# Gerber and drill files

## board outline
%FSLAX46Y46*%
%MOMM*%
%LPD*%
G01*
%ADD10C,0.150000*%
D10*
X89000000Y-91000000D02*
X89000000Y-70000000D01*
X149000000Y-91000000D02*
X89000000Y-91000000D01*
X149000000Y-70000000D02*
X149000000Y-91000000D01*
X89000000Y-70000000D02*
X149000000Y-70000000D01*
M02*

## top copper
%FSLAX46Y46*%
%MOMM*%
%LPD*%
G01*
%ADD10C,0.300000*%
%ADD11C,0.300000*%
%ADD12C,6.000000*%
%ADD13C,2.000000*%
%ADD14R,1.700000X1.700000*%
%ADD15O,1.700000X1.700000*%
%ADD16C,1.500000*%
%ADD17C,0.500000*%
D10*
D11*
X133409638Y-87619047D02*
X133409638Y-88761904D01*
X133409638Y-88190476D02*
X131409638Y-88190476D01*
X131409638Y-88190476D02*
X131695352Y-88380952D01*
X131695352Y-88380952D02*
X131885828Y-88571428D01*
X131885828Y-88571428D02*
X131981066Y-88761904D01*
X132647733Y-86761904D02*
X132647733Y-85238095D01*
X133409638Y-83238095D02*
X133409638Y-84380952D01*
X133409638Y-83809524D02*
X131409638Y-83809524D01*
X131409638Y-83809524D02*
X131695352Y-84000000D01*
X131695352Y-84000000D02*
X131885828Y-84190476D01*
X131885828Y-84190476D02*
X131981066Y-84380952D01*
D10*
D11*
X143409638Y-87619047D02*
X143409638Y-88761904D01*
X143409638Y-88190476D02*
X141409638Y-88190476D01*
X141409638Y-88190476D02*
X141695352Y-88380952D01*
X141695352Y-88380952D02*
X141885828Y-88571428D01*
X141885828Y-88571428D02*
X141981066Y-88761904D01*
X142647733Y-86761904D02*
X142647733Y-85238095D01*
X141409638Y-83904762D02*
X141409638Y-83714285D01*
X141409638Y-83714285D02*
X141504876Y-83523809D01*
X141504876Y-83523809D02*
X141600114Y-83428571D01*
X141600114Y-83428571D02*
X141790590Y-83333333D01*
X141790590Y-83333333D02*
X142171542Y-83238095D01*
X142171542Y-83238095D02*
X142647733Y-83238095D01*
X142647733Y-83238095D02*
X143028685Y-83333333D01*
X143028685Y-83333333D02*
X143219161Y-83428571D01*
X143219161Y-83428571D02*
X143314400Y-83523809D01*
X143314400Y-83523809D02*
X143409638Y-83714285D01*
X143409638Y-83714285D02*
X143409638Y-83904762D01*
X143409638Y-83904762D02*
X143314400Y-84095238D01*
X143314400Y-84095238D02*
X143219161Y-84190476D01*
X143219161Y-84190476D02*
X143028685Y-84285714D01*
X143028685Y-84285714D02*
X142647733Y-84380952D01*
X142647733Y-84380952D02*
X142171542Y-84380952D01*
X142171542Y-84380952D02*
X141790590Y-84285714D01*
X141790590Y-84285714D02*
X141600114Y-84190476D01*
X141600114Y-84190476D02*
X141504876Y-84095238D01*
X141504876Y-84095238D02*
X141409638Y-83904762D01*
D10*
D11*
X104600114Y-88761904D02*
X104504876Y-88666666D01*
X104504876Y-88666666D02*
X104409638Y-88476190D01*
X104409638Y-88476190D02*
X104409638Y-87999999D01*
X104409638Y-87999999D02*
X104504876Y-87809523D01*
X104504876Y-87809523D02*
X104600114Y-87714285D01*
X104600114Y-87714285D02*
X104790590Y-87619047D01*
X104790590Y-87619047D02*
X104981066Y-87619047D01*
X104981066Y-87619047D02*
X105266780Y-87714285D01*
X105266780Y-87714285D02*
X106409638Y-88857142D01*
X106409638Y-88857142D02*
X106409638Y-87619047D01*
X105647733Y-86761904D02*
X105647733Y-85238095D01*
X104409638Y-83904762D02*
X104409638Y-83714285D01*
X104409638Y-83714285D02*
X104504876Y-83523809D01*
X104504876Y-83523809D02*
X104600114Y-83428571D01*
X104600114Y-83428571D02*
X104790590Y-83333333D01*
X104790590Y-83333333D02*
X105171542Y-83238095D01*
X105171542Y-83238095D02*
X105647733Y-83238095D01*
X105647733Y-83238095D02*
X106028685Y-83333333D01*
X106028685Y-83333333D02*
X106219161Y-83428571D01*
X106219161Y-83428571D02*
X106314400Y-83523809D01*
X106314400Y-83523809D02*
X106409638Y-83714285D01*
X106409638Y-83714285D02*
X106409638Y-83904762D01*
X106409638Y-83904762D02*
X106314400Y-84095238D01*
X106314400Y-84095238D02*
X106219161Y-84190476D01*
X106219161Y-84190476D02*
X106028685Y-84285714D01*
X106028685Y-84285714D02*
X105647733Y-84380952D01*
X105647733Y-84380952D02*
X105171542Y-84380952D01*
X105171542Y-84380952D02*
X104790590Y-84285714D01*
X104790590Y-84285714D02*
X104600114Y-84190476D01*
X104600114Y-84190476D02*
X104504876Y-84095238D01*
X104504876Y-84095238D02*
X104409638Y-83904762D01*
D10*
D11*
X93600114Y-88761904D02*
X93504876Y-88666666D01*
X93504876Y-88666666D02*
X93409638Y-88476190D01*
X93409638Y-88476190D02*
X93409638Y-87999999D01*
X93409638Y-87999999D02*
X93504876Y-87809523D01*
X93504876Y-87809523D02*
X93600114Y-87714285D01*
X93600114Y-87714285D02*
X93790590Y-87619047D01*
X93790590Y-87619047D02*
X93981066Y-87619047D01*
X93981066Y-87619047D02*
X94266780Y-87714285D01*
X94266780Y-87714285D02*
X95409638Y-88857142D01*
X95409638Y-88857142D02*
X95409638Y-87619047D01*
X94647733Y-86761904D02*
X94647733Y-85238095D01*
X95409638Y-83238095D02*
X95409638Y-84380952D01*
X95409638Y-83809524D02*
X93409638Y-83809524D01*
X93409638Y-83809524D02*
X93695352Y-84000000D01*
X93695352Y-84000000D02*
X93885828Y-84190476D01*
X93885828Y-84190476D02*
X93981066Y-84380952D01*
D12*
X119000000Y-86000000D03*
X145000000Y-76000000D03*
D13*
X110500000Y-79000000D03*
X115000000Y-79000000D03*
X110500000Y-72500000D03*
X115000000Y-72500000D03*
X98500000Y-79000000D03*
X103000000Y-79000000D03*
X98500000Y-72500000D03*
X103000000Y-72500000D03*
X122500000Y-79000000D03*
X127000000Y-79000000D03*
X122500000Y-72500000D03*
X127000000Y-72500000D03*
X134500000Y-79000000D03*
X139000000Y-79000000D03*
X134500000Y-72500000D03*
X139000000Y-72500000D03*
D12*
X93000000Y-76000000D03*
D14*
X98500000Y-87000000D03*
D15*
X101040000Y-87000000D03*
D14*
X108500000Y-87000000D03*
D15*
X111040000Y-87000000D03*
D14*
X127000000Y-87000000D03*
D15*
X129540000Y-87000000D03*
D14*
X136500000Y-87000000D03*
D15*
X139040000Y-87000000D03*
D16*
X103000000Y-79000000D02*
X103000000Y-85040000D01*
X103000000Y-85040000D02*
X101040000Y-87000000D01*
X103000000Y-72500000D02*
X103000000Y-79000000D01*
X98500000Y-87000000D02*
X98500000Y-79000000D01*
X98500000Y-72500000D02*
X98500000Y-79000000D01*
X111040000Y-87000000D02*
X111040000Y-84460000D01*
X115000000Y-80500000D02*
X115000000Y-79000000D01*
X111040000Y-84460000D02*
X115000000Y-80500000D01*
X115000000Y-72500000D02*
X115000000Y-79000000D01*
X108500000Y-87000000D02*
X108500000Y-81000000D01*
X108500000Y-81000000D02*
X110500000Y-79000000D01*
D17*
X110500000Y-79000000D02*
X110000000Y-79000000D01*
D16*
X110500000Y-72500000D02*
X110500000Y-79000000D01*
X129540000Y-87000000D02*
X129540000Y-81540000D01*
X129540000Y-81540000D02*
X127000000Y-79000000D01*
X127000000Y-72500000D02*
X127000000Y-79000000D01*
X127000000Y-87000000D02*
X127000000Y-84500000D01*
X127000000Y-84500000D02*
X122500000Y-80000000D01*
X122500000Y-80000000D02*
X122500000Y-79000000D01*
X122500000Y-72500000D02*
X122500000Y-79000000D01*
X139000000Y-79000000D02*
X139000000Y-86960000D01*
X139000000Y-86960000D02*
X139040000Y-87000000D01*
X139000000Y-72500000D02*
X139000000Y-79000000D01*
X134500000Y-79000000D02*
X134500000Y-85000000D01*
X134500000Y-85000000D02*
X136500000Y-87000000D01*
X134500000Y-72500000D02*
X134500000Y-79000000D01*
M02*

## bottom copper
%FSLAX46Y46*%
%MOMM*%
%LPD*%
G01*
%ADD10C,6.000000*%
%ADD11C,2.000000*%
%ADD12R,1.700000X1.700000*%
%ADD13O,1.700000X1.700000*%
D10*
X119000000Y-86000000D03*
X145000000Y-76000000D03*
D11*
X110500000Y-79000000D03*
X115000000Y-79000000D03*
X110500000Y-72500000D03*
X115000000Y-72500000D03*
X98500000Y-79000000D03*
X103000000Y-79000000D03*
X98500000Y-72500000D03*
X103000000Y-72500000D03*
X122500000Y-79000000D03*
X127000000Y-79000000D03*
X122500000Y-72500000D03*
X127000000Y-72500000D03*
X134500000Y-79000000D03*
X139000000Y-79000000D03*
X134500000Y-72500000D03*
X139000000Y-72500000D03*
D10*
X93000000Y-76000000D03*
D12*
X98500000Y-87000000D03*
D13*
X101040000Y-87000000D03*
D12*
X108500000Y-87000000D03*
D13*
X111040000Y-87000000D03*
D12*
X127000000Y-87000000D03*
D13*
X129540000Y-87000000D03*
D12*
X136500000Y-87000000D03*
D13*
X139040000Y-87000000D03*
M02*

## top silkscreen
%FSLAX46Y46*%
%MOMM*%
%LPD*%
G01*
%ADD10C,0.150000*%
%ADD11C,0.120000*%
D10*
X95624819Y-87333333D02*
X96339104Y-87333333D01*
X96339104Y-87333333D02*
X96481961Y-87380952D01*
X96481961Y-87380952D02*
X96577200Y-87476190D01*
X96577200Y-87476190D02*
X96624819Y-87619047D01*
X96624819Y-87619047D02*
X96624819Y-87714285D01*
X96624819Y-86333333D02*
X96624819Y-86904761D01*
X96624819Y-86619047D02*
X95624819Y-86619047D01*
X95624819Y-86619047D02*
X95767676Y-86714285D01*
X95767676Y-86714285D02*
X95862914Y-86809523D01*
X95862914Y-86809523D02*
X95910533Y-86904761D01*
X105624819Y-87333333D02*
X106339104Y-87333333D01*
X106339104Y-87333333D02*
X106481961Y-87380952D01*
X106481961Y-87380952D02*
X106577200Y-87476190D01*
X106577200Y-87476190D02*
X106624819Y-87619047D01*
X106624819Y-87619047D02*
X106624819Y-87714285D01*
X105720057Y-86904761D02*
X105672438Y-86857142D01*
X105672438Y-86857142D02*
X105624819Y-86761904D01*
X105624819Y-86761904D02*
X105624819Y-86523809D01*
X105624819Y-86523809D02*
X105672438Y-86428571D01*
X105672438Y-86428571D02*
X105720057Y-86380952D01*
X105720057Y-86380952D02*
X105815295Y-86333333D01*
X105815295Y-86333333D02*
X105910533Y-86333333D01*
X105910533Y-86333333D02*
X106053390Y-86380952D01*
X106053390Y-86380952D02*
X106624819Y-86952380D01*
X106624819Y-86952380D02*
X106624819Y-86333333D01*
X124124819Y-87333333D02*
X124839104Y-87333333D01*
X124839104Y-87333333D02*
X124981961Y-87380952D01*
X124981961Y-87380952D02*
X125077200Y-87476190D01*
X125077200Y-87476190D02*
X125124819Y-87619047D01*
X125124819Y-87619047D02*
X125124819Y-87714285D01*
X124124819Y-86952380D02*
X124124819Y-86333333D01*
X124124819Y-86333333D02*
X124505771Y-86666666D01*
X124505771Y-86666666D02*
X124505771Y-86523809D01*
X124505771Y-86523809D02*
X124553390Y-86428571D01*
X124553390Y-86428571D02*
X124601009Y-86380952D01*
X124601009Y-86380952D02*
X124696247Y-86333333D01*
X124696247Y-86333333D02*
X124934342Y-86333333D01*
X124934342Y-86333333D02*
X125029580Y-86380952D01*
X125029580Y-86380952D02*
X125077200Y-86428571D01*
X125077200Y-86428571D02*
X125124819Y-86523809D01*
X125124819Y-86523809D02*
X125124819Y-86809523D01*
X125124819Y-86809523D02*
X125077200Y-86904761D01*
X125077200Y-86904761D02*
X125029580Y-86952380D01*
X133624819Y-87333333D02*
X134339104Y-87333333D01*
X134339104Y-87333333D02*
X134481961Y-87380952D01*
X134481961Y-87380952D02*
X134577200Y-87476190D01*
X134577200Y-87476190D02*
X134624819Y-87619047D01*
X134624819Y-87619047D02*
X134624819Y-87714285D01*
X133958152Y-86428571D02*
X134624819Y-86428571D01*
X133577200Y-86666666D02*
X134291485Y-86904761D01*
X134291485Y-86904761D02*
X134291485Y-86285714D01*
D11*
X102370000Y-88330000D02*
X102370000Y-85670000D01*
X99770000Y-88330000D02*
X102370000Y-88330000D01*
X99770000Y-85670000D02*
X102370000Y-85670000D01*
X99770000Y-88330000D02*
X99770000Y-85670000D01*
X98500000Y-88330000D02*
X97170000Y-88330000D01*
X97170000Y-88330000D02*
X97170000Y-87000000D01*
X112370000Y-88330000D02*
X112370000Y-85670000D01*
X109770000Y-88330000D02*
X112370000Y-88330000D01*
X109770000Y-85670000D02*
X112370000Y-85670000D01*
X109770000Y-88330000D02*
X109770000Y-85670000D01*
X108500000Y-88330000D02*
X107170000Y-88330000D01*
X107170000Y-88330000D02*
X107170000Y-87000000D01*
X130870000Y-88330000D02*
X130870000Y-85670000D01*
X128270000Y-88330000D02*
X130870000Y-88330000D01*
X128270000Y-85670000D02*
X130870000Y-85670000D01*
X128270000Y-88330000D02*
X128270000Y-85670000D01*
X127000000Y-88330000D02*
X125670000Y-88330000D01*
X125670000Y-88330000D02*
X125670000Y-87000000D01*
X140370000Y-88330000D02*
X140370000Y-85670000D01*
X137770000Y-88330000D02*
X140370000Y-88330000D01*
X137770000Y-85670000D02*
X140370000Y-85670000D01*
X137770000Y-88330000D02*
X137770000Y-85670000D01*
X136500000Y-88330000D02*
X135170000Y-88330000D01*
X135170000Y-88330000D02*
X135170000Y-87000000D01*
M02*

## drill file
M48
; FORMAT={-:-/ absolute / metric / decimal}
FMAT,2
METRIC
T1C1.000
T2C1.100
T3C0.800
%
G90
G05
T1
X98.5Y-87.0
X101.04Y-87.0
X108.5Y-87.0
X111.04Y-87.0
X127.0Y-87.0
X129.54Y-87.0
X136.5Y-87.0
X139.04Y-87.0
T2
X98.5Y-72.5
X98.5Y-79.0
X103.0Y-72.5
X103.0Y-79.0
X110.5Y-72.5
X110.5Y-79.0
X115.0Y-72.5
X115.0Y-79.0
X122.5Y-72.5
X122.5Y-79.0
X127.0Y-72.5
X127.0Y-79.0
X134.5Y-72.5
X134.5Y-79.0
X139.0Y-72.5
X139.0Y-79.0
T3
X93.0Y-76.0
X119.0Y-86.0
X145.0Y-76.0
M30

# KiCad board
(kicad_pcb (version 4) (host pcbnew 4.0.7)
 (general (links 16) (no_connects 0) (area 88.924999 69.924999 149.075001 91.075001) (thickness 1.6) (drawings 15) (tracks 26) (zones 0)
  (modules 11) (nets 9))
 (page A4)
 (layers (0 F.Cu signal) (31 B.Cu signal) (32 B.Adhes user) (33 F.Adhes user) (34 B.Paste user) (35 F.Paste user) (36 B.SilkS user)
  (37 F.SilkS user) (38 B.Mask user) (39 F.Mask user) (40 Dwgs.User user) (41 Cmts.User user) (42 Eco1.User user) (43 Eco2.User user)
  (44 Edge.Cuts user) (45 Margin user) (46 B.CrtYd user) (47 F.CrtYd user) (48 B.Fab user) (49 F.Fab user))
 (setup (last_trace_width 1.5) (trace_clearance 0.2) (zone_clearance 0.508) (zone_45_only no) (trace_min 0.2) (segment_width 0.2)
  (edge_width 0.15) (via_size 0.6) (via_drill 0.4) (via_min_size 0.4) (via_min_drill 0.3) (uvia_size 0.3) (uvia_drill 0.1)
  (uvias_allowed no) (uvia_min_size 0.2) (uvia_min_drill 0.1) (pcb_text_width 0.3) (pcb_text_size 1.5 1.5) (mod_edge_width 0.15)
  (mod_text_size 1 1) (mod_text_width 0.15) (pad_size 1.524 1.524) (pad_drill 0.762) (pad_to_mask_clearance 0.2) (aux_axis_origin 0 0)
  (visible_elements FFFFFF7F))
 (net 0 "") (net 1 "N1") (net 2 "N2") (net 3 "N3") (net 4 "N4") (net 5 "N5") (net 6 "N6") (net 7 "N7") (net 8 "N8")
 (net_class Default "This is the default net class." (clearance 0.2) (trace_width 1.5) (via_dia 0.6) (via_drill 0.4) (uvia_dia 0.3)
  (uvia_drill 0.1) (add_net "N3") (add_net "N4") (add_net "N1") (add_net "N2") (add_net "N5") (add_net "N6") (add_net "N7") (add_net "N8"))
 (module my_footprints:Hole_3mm (layer F.Cu) (at 119 86)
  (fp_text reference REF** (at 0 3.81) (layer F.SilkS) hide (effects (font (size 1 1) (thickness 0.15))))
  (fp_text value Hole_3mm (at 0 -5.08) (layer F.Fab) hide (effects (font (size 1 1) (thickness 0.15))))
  (pad "" np_thru_hole circle (at 0 0) (size 6 6) (drill 0.8) (layers *.Cu *.Mask)))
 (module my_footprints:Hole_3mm (layer F.Cu) (at 145 76)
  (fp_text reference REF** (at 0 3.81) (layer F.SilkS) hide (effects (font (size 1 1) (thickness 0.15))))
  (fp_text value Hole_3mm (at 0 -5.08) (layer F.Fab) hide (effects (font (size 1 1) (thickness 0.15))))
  (pad "" np_thru_hole circle (at 0 0) (size 6 6) (drill 0.8) (layers *.Cu *.Mask)))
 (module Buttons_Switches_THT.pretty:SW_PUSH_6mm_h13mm (layer B.Cu) (at 115 79 90)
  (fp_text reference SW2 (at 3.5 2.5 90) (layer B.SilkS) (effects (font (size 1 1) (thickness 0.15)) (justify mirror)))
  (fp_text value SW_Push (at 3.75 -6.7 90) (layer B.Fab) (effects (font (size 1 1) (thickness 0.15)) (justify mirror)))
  (pad 2 thru_hole circle (at 0 -4.5) (size 2 2) (drill 1.1) (layers *.Cu *.Mask) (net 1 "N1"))
  (pad 1 thru_hole circle (at 0 0) (size 2 2) (drill 1.1) (layers *.Cu *.Mask) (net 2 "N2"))
  (pad 2 thru_hole circle (at 6.5 -4.5) (size 2 2) (drill 1.1) (layers *.Cu *.Mask) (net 1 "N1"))
  (pad 1 thru_hole circle (at 6.5 0) (size 2 2) (drill 1.1) (layers *.Cu *.Mask) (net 2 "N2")))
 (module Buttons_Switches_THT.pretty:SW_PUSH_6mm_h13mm (layer B.Cu) (at 103 79 90)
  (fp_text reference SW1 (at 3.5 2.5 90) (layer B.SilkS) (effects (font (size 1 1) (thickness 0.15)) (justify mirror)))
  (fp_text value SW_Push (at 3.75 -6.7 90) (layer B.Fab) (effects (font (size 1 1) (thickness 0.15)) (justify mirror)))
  (pad 2 thru_hole circle (at 0 -4.5) (size 2 2) (drill 1.1) (layers *.Cu *.Mask) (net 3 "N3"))
  (pad 1 thru_hole circle (at 0 0) (size 2 2) (drill 1.1) (layers *.Cu *.Mask) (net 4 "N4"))
  (pad 2 thru_hole circle (at 6.5 -4.5) (size 2 2) (drill 1.1) (layers *.Cu *.Mask) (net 3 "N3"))
  (pad 1 thru_hole circle (at 6.5 0) (size 2 2) (drill 1.1) (layers *.Cu *.Mask) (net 4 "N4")))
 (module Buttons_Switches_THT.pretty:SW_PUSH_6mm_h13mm (layer B.Cu) (at 127 79 90)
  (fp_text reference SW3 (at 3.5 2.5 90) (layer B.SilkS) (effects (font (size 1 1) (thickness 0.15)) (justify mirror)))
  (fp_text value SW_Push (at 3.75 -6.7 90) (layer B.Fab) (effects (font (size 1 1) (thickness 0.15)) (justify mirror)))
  (pad 2 thru_hole circle (at 0 -4.5) (size 2 2) (drill 1.1) (layers *.Cu *.Mask) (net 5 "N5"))
  (pad 1 thru_hole circle (at 0 0) (size 2 2) (drill 1.1) (layers *.Cu *.Mask) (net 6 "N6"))
  (pad 2 thru_hole circle (at 6.5 -4.5) (size 2 2) (drill 1.1) (layers *.Cu *.Mask) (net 5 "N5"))
  (pad 1 thru_hole circle (at 6.5 0) (size 2 2) (drill 1.1) (layers *.Cu *.Mask) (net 6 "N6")))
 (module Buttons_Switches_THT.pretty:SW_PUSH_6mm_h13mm (layer B.Cu) (at 139 79 90)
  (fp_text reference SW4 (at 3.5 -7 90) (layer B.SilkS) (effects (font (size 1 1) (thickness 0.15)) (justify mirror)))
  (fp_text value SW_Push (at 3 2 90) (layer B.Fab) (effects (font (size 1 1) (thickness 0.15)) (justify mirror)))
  (pad 2 thru_hole circle (at 0 -4.5) (size 2 2) (drill 1.1) (layers *.Cu *.Mask) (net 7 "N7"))
  (pad 1 thru_hole circle (at 0 0) (size 2 2) (drill 1.1) (layers *.Cu *.Mask) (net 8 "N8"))
  (pad 2 thru_hole circle (at 6.5 -4.5) (size 2 2) (drill 1.1) (layers *.Cu *.Mask) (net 7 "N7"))
  (pad 1 thru_hole circle (at 6.5 0) (size 2 2) (drill 1.1) (layers *.Cu *.Mask) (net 8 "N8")))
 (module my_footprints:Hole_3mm (layer F.Cu) (at 93 76)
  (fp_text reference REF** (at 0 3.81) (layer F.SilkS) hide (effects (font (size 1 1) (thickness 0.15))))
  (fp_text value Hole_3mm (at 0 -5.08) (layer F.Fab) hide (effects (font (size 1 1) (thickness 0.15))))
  (pad "" np_thru_hole circle (at 0 0) (size 6 6) (drill 0.8) (layers *.Cu *.Mask)))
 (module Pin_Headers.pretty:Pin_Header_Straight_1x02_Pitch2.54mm (layer F.Cu) (at 98.5 87 90)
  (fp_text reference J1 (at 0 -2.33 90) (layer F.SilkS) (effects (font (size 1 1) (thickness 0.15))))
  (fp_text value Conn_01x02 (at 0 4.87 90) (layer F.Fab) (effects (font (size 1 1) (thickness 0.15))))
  (fp_line (start -1.33 3.87) (end 1.33 3.87) (layer F.SilkS) (width 0.12))
  (fp_line (start -1.33 1.27) (end -1.33 3.87) (layer F.SilkS) (width 0.12))
  (fp_line (start 1.33 1.27) (end 1.33 3.87) (layer F.SilkS) (width 0.12))
  (fp_line (start -1.33 1.27) (end 1.33 1.27) (layer F.SilkS) (width 0.12))
  (fp_line (start -1.33 0) (end -1.33 -1.33) (layer F.SilkS) (width 0.12))
  (fp_line (start -1.33 -1.33) (end 0 -1.33) (layer F.SilkS) (width 0.12))
  (pad 1 thru_hole rect (at 0 0 90) (size 1.7 1.7) (drill 1) (layers *.Cu *.Mask) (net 3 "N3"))
  (pad 2 thru_hole oval (at 0 2.54 90) (size 1.7 1.7) (drill 1) (layers *.Cu *.Mask) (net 4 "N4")))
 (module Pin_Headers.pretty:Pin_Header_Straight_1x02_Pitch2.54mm (layer F.Cu) (at 108.5 87 90)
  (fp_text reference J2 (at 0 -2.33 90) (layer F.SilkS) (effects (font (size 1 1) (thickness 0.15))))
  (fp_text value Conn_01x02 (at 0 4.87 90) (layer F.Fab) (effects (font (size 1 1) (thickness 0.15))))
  (fp_line (start -1.33 3.87) (end 1.33 3.87) (layer F.SilkS) (width 0.12))
  (fp_line (start -1.33 1.27) (end -1.33 3.87) (layer F.SilkS) (width 0.12))
  (fp_line (start 1.33 1.27) (end 1.33 3.87) (layer F.SilkS) (width 0.12))
  (fp_line (start -1.33 1.27) (end 1.33 1.27) (layer F.SilkS) (width 0.12))
  (fp_line (start -1.33 0) (end -1.33 -1.33) (layer F.SilkS) (width 0.12))
  (fp_line (start -1.33 -1.33) (end 0 -1.33) (layer F.SilkS) (width 0.12))
  (pad 1 thru_hole rect (at 0 0 90) (size 1.7 1.7) (drill 1) (layers *.Cu *.Mask) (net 1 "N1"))
  (pad 2 thru_hole oval (at 0 2.54 90) (size 1.7 1.7) (drill 1) (layers *.Cu *.Mask) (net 2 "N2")))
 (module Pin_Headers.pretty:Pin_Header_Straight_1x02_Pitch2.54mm (layer F.Cu) (at 127 87 90)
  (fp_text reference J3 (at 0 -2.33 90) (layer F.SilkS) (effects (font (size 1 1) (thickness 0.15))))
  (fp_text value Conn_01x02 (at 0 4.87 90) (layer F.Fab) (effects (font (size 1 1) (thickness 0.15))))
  (fp_line (start -1.33 3.87) (end 1.33 3.87) (layer F.SilkS) (width 0.12))
  (fp_line (start -1.33 1.27) (end -1.33 3.87) (layer F.SilkS) (width 0.12))
  (fp_line (start 1.33 1.27) (end 1.33 3.87) (layer F.SilkS) (width 0.12))
  (fp_line (start -1.33 1.27) (end 1.33 1.27) (layer F.SilkS) (width 0.12))
  (fp_line (start -1.33 0) (end -1.33 -1.33) (layer F.SilkS) (width 0.12))
  (fp_line (start -1.33 -1.33) (end 0 -1.33) (layer F.SilkS) (width 0.12))
  (pad 1 thru_hole rect (at 0 0 90) (size 1.7 1.7) (drill 1) (layers *.Cu *.Mask) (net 5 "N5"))
  (pad 2 thru_hole oval (at 0 2.54 90) (size 1.7 1.7) (drill 1) (layers *.Cu *.Mask) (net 6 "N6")))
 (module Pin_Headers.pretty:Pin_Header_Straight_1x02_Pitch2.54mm (layer F.Cu) (at 136.5 87 90)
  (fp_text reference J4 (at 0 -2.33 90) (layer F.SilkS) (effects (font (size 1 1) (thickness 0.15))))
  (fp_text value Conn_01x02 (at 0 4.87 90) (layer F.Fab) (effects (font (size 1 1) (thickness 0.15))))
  (fp_line (start -1.33 3.87) (end 1.33 3.87) (layer F.SilkS) (width 0.12))
  (fp_line (start -1.33 1.27) (end -1.33 3.87) (layer F.SilkS) (width 0.12))
  (fp_line (start 1.33 1.27) (end 1.33 3.87) (layer F.SilkS) (width 0.12))
  (fp_line (start -1.33 1.27) (end 1.33 1.27) (layer F.SilkS) (width 0.12))
  (fp_line (start -1.33 0) (end -1.33 -1.33) (layer F.SilkS) (width 0.12))
  (fp_line (start -1.33 -1.33) (end 0 -1.33) (layer F.SilkS) (width 0.12))
  (pad 1 thru_hole rect (at 0 0 90) (size 1.7 1.7) (drill 1) (layers *.Cu *.Mask) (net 7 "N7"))
  (pad 2 thru_hole oval (at 0 2.54 90) (size 1.7 1.7) (drill 1) (layers *.Cu *.Mask) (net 8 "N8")))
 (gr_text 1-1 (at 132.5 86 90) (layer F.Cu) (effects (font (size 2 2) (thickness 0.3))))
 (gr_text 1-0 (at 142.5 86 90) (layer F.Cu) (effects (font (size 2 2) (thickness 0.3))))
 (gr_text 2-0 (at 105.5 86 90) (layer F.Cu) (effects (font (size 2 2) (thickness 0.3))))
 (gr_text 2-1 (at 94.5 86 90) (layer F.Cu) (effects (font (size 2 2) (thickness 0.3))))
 (gr_line (start 89 91) (end 89 70) (angle 90) (layer Edge.Cuts) (width 0.15))
 (gr_line (start 149 91) (end 89 91) (angle 90) (layer Edge.Cuts) (width 0.15))
 (gr_line (start 149 70) (end 149 91) (angle 90) (layer Edge.Cuts) (width 0.15))
 (gr_line (start 89 70) (end 149 70) (angle 90) (layer Edge.Cuts) (width 0.15))
 (segment (start 103 79) (end 103 85.04) (width 1.5) (layer F.Cu) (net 4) (status 400000))
 (segment (start 103 85.04) (end 101.04 87) (width 1.5) (layer F.Cu) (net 4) (status 800000))
 (segment (start 103 72.5) (end 103 79) (width 1.5) (layer F.Cu) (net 4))
 (segment (start 98.5 87) (end 98.5 79) (width 1.5) (layer F.Cu) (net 3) (status C00000))
 (segment (start 98.5 72.5) (end 98.5 79) (width 1.5) (layer F.Cu) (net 3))
 (segment (start 111.04 87) (end 111.04 84.46) (width 1.5) (layer F.Cu) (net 2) (status 400000))
 (segment (start 115 80.5) (end 115 79) (width 1.5) (layer F.Cu) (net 2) (status 800000))
 (segment (start 111.04 84.46) (end 115 80.5) (width 1.5) (layer F.Cu) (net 2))
 (segment (start 115 72.5) (end 115 79) (width 1.5) (layer F.Cu) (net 2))
 (segment (start 108.5 87) (end 108.5 81) (width 1.5) (layer F.Cu) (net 1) (status 400000))
 (segment (start 108.5 81) (end 110.5 79) (width 1.5) (layer F.Cu) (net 1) (status 800000))
 (segment (start 110.5 79) (end 110 79) (width 0.5) (layer F.Cu) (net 1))
 (segment (start 110.5 72.5) (end 110.5 79) (width 1.5) (layer F.Cu) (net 1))
 (segment (start 129.54 87) (end 129.54 81.54) (width 1.5) (layer F.Cu) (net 6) (status 400000))
 (segment (start 129.54 81.54) (end 127 79) (width 1.5) (layer F.Cu) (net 6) (status 800000))
 (segment (start 127 72.5) (end 127 79) (width 1.5) (layer F.Cu) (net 6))
 (segment (start 127 87) (end 127 84.5) (width 1.5) (layer F.Cu) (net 5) (status 400000))
 (segment (start 127 84.5) (end 122.5 80) (width 1.5) (layer F.Cu) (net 5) (status 800000))
 (segment (start 122.5 80) (end 122.5 79) (width 1.5) (layer F.Cu) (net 5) (status C00000))
 (segment (start 122.5 72.5) (end 122.5 79) (width 1.5) (layer F.Cu) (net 5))
 (segment (start 139 79) (end 139 86.96) (width 1.5) (layer F.Cu) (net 8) (status C00000))
 (segment (start 139 86.96) (end 139.04 87) (width 1.5) (layer F.Cu) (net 8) (status C00000))
 (segment (start 139 72.5) (end 139 79) (width 1.5) (layer F.Cu) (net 8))
 (segment (start 134.5 79) (end 134.5 85) (width 1.5) (layer F.Cu) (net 7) (status 400000))
 (segment (start 134.5 85) (end 136.5 87) (width 1.5) (layer F.Cu) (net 7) (status 800000))
 (segment (start 134.5 72.5) (end 134.5 79) (width 1.5) (layer F.Cu) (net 7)))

